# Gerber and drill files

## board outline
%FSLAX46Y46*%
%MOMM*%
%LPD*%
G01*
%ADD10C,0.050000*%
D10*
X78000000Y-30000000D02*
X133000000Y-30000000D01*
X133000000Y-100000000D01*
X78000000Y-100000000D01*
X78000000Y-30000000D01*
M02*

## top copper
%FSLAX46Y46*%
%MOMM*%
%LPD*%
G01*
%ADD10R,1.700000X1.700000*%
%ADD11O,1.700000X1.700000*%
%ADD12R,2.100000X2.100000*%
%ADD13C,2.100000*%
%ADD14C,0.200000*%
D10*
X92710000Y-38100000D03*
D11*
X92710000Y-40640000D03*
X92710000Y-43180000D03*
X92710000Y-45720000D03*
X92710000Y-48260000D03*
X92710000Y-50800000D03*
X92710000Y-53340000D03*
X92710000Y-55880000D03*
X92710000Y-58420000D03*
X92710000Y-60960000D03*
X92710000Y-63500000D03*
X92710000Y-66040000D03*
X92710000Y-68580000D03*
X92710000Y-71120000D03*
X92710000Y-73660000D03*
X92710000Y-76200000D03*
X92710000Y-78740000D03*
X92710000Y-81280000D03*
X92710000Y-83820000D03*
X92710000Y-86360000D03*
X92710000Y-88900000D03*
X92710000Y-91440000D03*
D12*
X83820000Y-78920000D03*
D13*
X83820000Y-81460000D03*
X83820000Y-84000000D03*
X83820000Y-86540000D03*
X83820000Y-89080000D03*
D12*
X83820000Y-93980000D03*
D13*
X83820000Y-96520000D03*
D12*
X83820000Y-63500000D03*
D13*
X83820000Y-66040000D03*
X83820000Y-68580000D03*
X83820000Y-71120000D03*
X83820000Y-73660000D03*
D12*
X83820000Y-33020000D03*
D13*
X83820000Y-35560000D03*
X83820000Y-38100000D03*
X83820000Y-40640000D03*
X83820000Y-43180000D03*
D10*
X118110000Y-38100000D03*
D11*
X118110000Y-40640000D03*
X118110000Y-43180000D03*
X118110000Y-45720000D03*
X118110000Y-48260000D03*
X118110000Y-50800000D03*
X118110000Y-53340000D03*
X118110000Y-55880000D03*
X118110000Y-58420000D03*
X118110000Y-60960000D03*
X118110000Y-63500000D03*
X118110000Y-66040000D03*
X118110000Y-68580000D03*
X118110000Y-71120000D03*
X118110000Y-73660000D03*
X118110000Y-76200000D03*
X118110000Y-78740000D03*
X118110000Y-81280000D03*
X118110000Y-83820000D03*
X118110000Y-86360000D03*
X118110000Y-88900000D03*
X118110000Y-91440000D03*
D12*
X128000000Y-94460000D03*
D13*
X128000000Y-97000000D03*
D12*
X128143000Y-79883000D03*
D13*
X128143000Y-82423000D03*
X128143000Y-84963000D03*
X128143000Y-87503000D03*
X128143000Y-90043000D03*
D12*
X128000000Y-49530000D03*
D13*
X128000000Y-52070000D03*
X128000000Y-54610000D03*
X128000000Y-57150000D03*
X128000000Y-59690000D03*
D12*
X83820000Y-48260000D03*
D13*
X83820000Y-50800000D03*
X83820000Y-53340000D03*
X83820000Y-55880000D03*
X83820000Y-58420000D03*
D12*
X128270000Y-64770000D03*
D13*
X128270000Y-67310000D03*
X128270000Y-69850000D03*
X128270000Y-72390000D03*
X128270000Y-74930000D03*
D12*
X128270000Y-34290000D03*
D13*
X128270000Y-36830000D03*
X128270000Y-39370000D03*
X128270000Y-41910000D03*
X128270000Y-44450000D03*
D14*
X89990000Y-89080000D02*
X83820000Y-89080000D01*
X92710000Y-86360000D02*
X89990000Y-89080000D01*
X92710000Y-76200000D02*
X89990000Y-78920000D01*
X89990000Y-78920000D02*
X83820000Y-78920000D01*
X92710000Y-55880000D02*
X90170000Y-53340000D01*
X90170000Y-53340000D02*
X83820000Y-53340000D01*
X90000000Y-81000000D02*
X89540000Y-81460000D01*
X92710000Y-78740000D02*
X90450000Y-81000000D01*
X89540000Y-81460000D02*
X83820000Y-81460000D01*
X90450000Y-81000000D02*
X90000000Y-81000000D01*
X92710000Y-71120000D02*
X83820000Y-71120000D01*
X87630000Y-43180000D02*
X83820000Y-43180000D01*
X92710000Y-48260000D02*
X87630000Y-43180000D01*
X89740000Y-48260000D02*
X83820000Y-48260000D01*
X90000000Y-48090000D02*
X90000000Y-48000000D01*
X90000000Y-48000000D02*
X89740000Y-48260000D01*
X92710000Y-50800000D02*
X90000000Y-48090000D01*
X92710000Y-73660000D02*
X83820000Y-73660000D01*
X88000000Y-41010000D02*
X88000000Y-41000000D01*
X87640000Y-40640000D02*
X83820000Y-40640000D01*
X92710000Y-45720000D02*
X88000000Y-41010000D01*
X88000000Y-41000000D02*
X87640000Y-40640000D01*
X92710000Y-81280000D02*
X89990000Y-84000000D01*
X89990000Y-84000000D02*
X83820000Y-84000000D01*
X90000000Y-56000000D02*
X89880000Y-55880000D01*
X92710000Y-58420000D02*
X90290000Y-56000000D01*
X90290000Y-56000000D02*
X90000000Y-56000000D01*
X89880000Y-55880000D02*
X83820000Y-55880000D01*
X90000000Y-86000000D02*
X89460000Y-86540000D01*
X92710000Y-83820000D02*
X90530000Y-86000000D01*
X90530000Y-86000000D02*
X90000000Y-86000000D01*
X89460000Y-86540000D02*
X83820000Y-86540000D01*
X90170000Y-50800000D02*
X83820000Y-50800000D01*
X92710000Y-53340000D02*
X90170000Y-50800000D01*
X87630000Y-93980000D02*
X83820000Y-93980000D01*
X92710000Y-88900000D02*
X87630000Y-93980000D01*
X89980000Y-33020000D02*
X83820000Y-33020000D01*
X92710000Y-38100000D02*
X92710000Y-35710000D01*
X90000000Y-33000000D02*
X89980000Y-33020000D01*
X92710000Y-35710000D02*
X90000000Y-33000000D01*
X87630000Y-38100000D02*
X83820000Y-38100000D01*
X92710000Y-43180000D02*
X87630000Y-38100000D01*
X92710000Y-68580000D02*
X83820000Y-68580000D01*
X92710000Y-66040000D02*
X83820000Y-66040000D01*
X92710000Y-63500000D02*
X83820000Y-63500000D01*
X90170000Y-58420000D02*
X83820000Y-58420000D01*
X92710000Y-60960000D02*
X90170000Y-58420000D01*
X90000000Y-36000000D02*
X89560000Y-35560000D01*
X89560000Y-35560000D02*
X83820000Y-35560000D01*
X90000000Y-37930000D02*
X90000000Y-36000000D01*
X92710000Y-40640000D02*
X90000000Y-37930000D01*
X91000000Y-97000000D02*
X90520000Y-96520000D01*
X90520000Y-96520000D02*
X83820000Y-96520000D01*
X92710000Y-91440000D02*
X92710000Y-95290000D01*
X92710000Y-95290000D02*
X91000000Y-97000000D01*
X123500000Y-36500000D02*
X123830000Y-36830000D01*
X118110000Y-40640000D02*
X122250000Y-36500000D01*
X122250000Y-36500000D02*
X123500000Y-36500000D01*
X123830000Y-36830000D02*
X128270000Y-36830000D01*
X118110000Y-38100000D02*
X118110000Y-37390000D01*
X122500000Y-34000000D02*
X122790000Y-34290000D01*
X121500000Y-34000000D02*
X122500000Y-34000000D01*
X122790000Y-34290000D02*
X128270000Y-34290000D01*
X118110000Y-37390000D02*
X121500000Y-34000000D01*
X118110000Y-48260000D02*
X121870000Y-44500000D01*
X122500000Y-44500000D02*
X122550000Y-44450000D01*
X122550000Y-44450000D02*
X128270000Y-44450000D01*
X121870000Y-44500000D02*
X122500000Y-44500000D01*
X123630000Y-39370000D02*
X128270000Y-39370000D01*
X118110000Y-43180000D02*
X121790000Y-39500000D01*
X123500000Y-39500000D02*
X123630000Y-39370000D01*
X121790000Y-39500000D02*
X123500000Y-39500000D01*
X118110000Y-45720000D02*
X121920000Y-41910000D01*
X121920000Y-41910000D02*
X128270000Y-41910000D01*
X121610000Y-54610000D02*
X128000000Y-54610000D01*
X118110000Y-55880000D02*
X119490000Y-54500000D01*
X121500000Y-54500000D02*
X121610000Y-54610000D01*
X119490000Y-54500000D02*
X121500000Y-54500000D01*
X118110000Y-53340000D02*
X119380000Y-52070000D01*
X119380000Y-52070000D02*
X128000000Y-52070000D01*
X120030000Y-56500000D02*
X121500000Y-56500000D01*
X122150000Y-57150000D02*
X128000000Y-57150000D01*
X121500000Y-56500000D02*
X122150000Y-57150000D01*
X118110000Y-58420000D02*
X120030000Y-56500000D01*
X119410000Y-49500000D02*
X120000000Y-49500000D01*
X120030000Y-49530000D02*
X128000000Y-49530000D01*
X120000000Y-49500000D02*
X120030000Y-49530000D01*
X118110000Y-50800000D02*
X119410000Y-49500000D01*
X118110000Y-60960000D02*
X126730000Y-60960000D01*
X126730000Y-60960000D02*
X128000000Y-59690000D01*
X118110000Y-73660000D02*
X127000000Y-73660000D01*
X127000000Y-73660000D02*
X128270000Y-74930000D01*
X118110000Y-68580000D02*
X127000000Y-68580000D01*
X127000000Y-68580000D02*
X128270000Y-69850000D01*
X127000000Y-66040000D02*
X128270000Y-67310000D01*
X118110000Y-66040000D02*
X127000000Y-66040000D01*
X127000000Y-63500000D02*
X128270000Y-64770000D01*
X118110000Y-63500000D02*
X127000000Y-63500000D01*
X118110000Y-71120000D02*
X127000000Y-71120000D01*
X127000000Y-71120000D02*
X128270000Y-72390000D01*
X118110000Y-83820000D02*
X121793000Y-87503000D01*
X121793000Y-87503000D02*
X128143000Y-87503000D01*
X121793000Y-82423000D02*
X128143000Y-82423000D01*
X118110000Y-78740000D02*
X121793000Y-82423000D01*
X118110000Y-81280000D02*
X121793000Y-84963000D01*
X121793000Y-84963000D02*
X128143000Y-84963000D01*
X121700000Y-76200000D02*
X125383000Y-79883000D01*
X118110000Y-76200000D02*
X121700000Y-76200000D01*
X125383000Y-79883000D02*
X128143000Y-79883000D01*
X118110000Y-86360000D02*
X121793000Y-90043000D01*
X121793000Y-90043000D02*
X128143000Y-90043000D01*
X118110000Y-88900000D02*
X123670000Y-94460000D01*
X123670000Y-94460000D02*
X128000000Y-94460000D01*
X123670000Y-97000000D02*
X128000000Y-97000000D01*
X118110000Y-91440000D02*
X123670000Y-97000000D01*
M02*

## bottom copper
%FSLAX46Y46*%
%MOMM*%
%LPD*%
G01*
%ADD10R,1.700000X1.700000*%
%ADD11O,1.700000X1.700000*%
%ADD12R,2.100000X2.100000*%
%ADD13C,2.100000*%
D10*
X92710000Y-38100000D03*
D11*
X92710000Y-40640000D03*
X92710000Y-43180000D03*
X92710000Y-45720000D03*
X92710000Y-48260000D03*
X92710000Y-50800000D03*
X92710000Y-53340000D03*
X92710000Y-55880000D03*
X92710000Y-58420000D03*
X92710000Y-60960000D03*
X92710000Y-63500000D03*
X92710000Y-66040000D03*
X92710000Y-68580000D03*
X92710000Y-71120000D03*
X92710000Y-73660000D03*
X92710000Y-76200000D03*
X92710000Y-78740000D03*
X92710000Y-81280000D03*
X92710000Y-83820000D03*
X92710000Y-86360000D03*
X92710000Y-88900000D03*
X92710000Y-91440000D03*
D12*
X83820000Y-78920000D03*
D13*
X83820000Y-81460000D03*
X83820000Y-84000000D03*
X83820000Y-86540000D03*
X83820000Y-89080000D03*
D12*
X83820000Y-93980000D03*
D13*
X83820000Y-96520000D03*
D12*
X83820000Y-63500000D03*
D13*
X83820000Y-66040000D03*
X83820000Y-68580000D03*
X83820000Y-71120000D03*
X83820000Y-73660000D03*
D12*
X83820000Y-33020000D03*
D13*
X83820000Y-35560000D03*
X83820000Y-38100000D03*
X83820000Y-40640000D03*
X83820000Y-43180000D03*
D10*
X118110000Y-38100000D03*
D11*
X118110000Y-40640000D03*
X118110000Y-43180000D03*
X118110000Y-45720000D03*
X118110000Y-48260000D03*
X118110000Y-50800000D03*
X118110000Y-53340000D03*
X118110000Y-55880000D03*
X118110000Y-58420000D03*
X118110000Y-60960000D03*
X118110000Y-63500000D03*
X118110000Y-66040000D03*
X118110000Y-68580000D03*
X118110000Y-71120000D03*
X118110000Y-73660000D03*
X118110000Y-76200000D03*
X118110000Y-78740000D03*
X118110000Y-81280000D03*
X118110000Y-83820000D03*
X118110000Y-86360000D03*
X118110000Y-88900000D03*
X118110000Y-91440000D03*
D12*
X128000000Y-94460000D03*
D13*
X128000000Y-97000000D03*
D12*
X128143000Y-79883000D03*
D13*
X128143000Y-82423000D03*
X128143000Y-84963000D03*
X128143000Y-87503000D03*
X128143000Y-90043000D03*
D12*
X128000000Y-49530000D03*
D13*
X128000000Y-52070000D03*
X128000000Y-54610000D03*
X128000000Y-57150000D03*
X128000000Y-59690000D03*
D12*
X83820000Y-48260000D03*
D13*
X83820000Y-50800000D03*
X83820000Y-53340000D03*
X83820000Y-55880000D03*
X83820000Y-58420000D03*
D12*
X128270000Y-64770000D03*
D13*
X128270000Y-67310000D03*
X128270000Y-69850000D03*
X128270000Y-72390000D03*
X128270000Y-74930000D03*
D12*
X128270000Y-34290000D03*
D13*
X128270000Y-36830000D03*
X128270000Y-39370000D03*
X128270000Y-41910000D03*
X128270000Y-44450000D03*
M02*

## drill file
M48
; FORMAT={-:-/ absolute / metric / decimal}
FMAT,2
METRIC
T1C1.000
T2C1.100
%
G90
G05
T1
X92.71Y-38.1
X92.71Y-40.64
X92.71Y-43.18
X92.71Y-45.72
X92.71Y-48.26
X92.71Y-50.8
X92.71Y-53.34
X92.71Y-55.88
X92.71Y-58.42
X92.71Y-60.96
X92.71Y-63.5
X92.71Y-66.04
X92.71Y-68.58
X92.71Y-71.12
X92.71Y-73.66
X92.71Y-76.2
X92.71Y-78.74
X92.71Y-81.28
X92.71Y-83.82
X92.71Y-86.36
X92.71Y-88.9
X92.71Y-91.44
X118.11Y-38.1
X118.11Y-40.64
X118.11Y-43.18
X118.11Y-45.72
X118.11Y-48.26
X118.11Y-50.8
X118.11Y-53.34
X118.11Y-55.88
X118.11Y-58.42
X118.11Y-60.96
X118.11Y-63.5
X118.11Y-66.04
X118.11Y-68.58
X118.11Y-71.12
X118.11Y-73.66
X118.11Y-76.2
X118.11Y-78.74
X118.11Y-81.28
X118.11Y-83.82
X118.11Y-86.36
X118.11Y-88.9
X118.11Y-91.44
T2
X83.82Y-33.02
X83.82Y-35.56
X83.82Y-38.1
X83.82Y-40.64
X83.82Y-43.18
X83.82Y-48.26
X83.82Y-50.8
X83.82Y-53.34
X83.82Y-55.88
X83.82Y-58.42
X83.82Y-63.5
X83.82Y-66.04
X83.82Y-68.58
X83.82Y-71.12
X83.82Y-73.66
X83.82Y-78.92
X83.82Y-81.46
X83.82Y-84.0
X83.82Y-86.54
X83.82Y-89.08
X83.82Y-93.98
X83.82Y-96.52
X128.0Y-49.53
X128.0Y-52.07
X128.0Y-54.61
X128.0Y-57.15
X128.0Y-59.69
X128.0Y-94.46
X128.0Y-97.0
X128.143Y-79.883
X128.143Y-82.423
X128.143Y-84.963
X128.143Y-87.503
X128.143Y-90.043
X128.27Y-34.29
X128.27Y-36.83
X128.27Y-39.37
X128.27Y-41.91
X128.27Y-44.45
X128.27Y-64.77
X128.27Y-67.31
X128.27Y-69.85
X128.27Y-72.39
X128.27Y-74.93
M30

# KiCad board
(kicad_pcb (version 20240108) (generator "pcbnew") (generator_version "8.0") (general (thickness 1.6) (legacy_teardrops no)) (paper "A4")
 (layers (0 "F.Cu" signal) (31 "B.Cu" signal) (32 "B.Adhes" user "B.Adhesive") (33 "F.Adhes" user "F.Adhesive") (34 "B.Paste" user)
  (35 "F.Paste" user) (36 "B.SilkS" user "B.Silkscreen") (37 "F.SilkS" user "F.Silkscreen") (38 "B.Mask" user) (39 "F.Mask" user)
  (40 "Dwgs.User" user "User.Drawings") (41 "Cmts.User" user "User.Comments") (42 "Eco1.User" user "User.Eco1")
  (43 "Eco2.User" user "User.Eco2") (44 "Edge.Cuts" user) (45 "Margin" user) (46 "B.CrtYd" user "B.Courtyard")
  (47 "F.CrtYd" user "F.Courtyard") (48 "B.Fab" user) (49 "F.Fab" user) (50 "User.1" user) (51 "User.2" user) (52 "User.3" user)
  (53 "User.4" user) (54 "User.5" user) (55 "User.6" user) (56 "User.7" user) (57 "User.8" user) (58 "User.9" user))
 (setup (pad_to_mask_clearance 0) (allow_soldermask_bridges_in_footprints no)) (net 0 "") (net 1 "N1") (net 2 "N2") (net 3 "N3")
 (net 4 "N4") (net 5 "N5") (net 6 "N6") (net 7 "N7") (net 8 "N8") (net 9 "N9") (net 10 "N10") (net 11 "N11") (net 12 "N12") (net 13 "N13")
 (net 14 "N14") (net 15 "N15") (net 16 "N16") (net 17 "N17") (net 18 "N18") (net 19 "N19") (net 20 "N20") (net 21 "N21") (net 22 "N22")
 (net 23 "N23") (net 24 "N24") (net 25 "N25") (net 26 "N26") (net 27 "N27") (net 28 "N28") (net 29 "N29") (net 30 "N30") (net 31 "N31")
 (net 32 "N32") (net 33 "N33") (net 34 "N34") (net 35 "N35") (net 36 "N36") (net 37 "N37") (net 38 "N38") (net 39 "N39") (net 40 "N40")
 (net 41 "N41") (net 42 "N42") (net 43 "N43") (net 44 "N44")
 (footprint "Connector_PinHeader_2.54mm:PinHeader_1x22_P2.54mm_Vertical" (layer "F.Cu") (at 92.71 38.1)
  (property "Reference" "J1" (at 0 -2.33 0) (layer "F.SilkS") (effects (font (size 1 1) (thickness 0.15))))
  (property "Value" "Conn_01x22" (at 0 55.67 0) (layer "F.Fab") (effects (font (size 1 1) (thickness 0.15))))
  (pad "1" thru_hole rect (at 0 0) (size 1.7 1.7) (drill 1) (layers "*.Cu" "*.Mask") (remove_unused_layers no) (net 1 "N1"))
  (pad "2" thru_hole oval (at 0 2.54) (size 1.7 1.7) (drill 1) (layers "*.Cu" "*.Mask") (remove_unused_layers no) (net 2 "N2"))
  (pad "3" thru_hole oval (at 0 5.08) (size 1.7 1.7) (drill 1) (layers "*.Cu" "*.Mask") (remove_unused_layers no) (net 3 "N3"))
  (pad "4" thru_hole oval (at 0 7.62) (size 1.7 1.7) (drill 1) (layers "*.Cu" "*.Mask") (remove_unused_layers no) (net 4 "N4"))
  (pad "5" thru_hole oval (at 0 10.16) (size 1.7 1.7) (drill 1) (layers "*.Cu" "*.Mask") (remove_unused_layers no) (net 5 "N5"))
  (pad "6" thru_hole oval (at 0 12.7) (size 1.7 1.7) (drill 1) (layers "*.Cu" "*.Mask") (remove_unused_layers no) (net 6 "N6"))
  (pad "7" thru_hole oval (at 0 15.24) (size 1.7 1.7) (drill 1) (layers "*.Cu" "*.Mask") (remove_unused_layers no) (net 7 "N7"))
  (pad "8" thru_hole oval (at 0 17.78) (size 1.7 1.7) (drill 1) (layers "*.Cu" "*.Mask") (remove_unused_layers no) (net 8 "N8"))
  (pad "9" thru_hole oval (at 0 20.32) (size 1.7 1.7) (drill 1) (layers "*.Cu" "*.Mask") (remove_unused_layers no) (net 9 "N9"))
  (pad "10" thru_hole oval (at 0 22.86) (size 1.7 1.7) (drill 1) (layers "*.Cu" "*.Mask") (remove_unused_layers no) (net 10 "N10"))
  (pad "11" thru_hole oval (at 0 25.4) (size 1.7 1.7) (drill 1) (layers "*.Cu" "*.Mask") (remove_unused_layers no) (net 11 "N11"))
  (pad "12" thru_hole oval (at 0 27.94) (size 1.7 1.7) (drill 1) (layers "*.Cu" "*.Mask") (remove_unused_layers no) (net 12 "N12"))
  (pad "13" thru_hole oval (at 0 30.48) (size 1.7 1.7) (drill 1) (layers "*.Cu" "*.Mask") (remove_unused_layers no) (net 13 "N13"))
  (pad "14" thru_hole oval (at 0 33.02) (size 1.7 1.7) (drill 1) (layers "*.Cu" "*.Mask") (remove_unused_layers no) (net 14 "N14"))
  (pad "15" thru_hole oval (at 0 35.56) (size 1.7 1.7) (drill 1) (layers "*.Cu" "*.Mask") (remove_unused_layers no) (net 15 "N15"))
  (pad "16" thru_hole oval (at 0 38.1) (size 1.7 1.7) (drill 1) (layers "*.Cu" "*.Mask") (remove_unused_layers no) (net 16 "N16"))
  (pad "17" thru_hole oval (at 0 40.64) (size 1.7 1.7) (drill 1) (layers "*.Cu" "*.Mask") (remove_unused_layers no) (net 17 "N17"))
  (pad "18" thru_hole oval (at 0 43.18) (size 1.7 1.7) (drill 1) (layers "*.Cu" "*.Mask") (remove_unused_layers no) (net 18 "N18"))
  (pad "19" thru_hole oval (at 0 45.72) (size 1.7 1.7) (drill 1) (layers "*.Cu" "*.Mask") (remove_unused_layers no) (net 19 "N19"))
  (pad "20" thru_hole oval (at 0 48.26) (size 1.7 1.7) (drill 1) (layers "*.Cu" "*.Mask") (remove_unused_layers no) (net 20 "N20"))
  (pad "21" thru_hole oval (at 0 50.8) (size 1.7 1.7) (drill 1) (layers "*.Cu" "*.Mask") (remove_unused_layers no) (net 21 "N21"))
  (pad "22" thru_hole oval (at 0 53.34) (size 1.7 1.7) (drill 1) (layers "*.Cu" "*.Mask") (remove_unused_layers no) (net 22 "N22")))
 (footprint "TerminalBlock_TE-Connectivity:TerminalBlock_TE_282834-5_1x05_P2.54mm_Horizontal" (layer "F.Cu") (at 83.82 78.92 -90)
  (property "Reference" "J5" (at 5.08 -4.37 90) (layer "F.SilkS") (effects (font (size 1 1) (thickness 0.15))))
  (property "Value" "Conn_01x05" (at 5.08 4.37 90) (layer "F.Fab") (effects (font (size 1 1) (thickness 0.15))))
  (pad "1" thru_hole rect (at 0 0 270) (size 2.1 2.1) (drill 1.1) (layers "*.Cu" "*.Mask") (remove_unused_layers no) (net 16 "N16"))
  (pad "2" thru_hole circle (at 2.54 0 270) (size 2.1 2.1) (drill 1.1) (layers "*.Cu" "*.Mask") (remove_unused_layers no) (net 17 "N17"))
  (pad "3" thru_hole circle (at 5.08 0 270) (size 2.1 2.1) (drill 1.1) (layers "*.Cu" "*.Mask") (remove_unused_layers no) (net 18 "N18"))
  (pad "4" thru_hole circle (at 7.62 0 270) (size 2.1 2.1) (drill 1.1) (layers "*.Cu" "*.Mask") (remove_unused_layers no) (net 19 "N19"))
  (pad "5" thru_hole circle (at 10.16 0 270) (size 2.1 2.1) (drill 1.1) (layers "*.Cu" "*.Mask") (remove_unused_layers no) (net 20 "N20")))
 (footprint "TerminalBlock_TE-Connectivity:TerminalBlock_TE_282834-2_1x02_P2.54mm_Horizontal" (layer "F.Cu") (at 83.82 93.98 -90)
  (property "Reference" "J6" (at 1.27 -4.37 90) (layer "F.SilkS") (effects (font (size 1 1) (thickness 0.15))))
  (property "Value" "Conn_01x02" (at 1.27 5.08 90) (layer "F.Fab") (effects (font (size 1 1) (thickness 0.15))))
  (pad "1" thru_hole rect (at 0 0 270) (size 2.1 2.1) (drill 1.1) (layers "*.Cu" "*.Mask") (remove_unused_layers no) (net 21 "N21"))
  (pad "2" thru_hole circle (at 2.54 0 270) (size 2.1 2.1) (drill 1.1) (layers "*.Cu" "*.Mask") (remove_unused_layers no) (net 22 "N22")))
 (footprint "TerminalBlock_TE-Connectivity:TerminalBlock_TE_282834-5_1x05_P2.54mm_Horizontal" (layer "F.Cu") (at 83.82 63.5 -90)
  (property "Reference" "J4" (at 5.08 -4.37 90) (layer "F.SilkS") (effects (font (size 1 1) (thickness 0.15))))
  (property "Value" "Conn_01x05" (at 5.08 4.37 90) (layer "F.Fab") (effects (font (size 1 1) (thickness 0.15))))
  (pad "1" thru_hole rect (at 0 0 270) (size 2.1 2.1) (drill 1.1) (layers "*.Cu" "*.Mask") (remove_unused_layers no) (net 11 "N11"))
  (pad "2" thru_hole circle (at 2.54 0 270) (size 2.1 2.1) (drill 1.1) (layers "*.Cu" "*.Mask") (remove_unused_layers no) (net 12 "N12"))
  (pad "3" thru_hole circle (at 5.08 0 270) (size 2.1 2.1) (drill 1.1) (layers "*.Cu" "*.Mask") (remove_unused_layers no) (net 13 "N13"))
  (pad "4" thru_hole circle (at 7.62 0 270) (size 2.1 2.1) (drill 1.1) (layers "*.Cu" "*.Mask") (remove_unused_layers no) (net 14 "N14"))
  (pad "5" thru_hole circle (at 10.16 0 270) (size 2.1 2.1) (drill 1.1) (layers "*.Cu" "*.Mask") (remove_unused_layers no) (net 15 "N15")))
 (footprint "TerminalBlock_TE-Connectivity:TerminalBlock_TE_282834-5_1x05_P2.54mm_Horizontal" (layer "F.Cu") (at 83.82 33.02 -90)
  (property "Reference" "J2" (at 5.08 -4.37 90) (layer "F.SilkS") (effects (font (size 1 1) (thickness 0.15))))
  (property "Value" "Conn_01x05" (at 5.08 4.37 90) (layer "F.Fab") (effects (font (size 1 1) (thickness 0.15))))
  (pad "1" thru_hole rect (at 0 0 270) (size 2.1 2.1) (drill 1.1) (layers "*.Cu" "*.Mask") (remove_unused_layers no) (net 1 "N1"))
  (pad "2" thru_hole circle (at 2.54 0 270) (size 2.1 2.1) (drill 1.1) (layers "*.Cu" "*.Mask") (remove_unused_layers no) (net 2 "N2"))
  (pad "3" thru_hole circle (at 5.08 0 270) (size 2.1 2.1) (drill 1.1) (layers "*.Cu" "*.Mask") (remove_unused_layers no) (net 3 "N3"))
  (pad "4" thru_hole circle (at 7.62 0 270) (size 2.1 2.1) (drill 1.1) (layers "*.Cu" "*.Mask") (remove_unused_layers no) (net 4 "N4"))
  (pad "5" thru_hole circle (at 10.16 0 270) (size 2.1 2.1) (drill 1.1) (layers "*.Cu" "*.Mask") (remove_unused_layers no) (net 5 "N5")))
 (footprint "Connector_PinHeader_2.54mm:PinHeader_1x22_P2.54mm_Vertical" (layer "F.Cu") (at 118.11 38.1)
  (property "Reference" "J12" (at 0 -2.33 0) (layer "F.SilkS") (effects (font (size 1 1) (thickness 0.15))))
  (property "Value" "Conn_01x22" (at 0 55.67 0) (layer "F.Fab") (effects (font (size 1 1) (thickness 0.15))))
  (pad "1" thru_hole rect (at 0 0) (size 1.7 1.7) (drill 1) (layers "*.Cu" "*.Mask") (remove_unused_layers no) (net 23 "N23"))
  (pad "2" thru_hole oval (at 0 2.54) (size 1.7 1.7) (drill 1) (layers "*.Cu" "*.Mask") (remove_unused_layers no) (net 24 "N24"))
  (pad "3" thru_hole oval (at 0 5.08) (size 1.7 1.7) (drill 1) (layers "*.Cu" "*.Mask") (remove_unused_layers no) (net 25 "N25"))
  (pad "4" thru_hole oval (at 0 7.62) (size 1.7 1.7) (drill 1) (layers "*.Cu" "*.Mask") (remove_unused_layers no) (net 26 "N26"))
  (pad "5" thru_hole oval (at 0 10.16) (size 1.7 1.7) (drill 1) (layers "*.Cu" "*.Mask") (remove_unused_layers no) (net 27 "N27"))
  (pad "6" thru_hole oval (at 0 12.7) (size 1.7 1.7) (drill 1) (layers "*.Cu" "*.Mask") (remove_unused_layers no) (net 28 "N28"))
  (pad "7" thru_hole oval (at 0 15.24) (size 1.7 1.7) (drill 1) (layers "*.Cu" "*.Mask") (remove_unused_layers no) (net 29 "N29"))
  (pad "8" thru_hole oval (at 0 17.78) (size 1.7 1.7) (drill 1) (layers "*.Cu" "*.Mask") (remove_unused_layers no) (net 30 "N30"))
  (pad "9" thru_hole oval (at 0 20.32) (size 1.7 1.7) (drill 1) (layers "*.Cu" "*.Mask") (remove_unused_layers no) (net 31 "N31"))
  (pad "10" thru_hole oval (at 0 22.86) (size 1.7 1.7) (drill 1) (layers "*.Cu" "*.Mask") (remove_unused_layers no) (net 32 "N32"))
  (pad "11" thru_hole oval (at 0 25.4) (size 1.7 1.7) (drill 1) (layers "*.Cu" "*.Mask") (remove_unused_layers no) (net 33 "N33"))
  (pad "12" thru_hole oval (at 0 27.94) (size 1.7 1.7) (drill 1) (layers "*.Cu" "*.Mask") (remove_unused_layers no) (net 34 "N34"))
  (pad "13" thru_hole oval (at 0 30.48) (size 1.7 1.7) (drill 1) (layers "*.Cu" "*.Mask") (remove_unused_layers no) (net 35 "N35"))
  (pad "14" thru_hole oval (at 0 33.02) (size 1.7 1.7) (drill 1) (layers "*.Cu" "*.Mask") (remove_unused_layers no) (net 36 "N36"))
  (pad "15" thru_hole oval (at 0 35.56) (size 1.7 1.7) (drill 1) (layers "*.Cu" "*.Mask") (remove_unused_layers no) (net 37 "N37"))
  (pad "16" thru_hole oval (at 0 38.1) (size 1.7 1.7) (drill 1) (layers "*.Cu" "*.Mask") (remove_unused_layers no) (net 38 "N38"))
  (pad "17" thru_hole oval (at 0 40.64) (size 1.7 1.7) (drill 1) (layers "*.Cu" "*.Mask") (remove_unused_layers no) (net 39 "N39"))
  (pad "18" thru_hole oval (at 0 43.18) (size 1.7 1.7) (drill 1) (layers "*.Cu" "*.Mask") (remove_unused_layers no) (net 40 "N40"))
  (pad "19" thru_hole oval (at 0 45.72) (size 1.7 1.7) (drill 1) (layers "*.Cu" "*.Mask") (remove_unused_layers no) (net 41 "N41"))
  (pad "20" thru_hole oval (at 0 48.26) (size 1.7 1.7) (drill 1) (layers "*.Cu" "*.Mask") (remove_unused_layers no) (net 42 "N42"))
  (pad "21" thru_hole oval (at 0 50.8) (size 1.7 1.7) (drill 1) (layers "*.Cu" "*.Mask") (remove_unused_layers no) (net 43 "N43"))
  (pad "22" thru_hole oval (at 0 53.34) (size 1.7 1.7) (drill 1) (layers "*.Cu" "*.Mask") (remove_unused_layers no) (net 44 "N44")))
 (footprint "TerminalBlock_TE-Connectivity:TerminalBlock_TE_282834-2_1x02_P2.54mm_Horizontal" (layer "F.Cu") (at 128 94.46 -90)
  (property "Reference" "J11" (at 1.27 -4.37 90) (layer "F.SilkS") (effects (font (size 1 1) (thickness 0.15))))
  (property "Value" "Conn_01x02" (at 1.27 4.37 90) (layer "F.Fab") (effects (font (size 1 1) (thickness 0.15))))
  (pad "1" thru_hole rect (at 0 0 270) (size 2.1 2.1) (drill 1.1) (layers "*.Cu" "*.Mask") (remove_unused_layers no) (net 43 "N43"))
  (pad "2" thru_hole circle (at 2.54 0 270) (size 2.1 2.1) (drill 1.1) (layers "*.Cu" "*.Mask") (remove_unused_layers no) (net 44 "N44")))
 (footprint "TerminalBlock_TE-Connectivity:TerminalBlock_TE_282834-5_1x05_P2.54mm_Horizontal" (layer "F.Cu") (at 128.143 79.883 -90)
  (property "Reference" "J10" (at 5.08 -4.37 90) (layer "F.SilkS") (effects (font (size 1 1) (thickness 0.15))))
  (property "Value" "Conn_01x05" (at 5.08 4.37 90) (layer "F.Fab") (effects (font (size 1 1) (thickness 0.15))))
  (pad "1" thru_hole rect (at 0 0 270) (size 2.1 2.1) (drill 1.1) (layers "*.Cu" "*.Mask") (remove_unused_layers no) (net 38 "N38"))
  (pad "2" thru_hole circle (at 2.54 0 270) (size 2.1 2.1) (drill 1.1) (layers "*.Cu" "*.Mask") (remove_unused_layers no) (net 39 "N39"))
  (pad "3" thru_hole circle (at 5.08 0 270) (size 2.1 2.1) (drill 1.1) (layers "*.Cu" "*.Mask") (remove_unused_layers no) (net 40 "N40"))
  (pad "4" thru_hole circle (at 7.62 0 270) (size 2.1 2.1) (drill 1.1) (layers "*.Cu" "*.Mask") (remove_unused_layers no) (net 41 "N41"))
  (pad "5" thru_hole circle (at 10.16 0 270) (size 2.1 2.1) (drill 1.1) (layers "*.Cu" "*.Mask") (remove_unused_layers no) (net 42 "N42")))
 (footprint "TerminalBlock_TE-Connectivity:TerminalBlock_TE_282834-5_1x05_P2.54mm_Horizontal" (layer "F.Cu") (at 128 49.53 -90)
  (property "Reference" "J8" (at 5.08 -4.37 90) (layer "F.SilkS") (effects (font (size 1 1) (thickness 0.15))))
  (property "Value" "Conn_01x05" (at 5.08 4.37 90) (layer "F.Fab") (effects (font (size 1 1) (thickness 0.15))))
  (pad "1" thru_hole rect (at 0 0 270) (size 2.1 2.1) (drill 1.1) (layers "*.Cu" "*.Mask") (remove_unused_layers no) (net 28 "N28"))
  (pad "2" thru_hole circle (at 2.54 0 270) (size 2.1 2.1) (drill 1.1) (layers "*.Cu" "*.Mask") (remove_unused_layers no) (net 29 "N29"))
  (pad "3" thru_hole circle (at 5.08 0 270) (size 2.1 2.1) (drill 1.1) (layers "*.Cu" "*.Mask") (remove_unused_layers no) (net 30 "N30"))
  (pad "4" thru_hole circle (at 7.62 0 270) (size 2.1 2.1) (drill 1.1) (layers "*.Cu" "*.Mask") (remove_unused_layers no) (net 31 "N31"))
  (pad "5" thru_hole circle (at 10.16 0 270) (size 2.1 2.1) (drill 1.1) (layers "*.Cu" "*.Mask") (remove_unused_layers no) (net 32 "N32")))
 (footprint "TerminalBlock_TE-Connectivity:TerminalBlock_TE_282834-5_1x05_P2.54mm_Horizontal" (layer "F.Cu") (at 83.82 48.26 -90)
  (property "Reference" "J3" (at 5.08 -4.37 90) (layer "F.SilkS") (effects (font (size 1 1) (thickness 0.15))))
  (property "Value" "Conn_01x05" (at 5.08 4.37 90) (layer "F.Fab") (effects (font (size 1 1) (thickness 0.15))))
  (pad "1" thru_hole rect (at 0 0 270) (size 2.1 2.1) (drill 1.1) (layers "*.Cu" "*.Mask") (remove_unused_layers no) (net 6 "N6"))
  (pad "2" thru_hole circle (at 2.54 0 270) (size 2.1 2.1) (drill 1.1) (layers "*.Cu" "*.Mask") (remove_unused_layers no) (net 7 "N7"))
  (pad "3" thru_hole circle (at 5.08 0 270) (size 2.1 2.1) (drill 1.1) (layers "*.Cu" "*.Mask") (remove_unused_layers no) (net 8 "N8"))
  (pad "4" thru_hole circle (at 7.62 0 270) (size 2.1 2.1) (drill 1.1) (layers "*.Cu" "*.Mask") (remove_unused_layers no) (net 9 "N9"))
  (pad "5" thru_hole circle (at 10.16 0 270) (size 2.1 2.1) (drill 1.1) (layers "*.Cu" "*.Mask") (remove_unused_layers no) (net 10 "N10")))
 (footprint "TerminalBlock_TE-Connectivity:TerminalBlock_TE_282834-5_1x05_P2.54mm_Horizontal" (layer "F.Cu") (at 128.27 64.77 -90)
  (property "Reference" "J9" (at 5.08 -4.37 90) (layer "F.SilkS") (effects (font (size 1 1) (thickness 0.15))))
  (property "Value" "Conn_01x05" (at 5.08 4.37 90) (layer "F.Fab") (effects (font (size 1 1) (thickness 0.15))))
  (pad "1" thru_hole rect (at 0 0 270) (size 2.1 2.1) (drill 1.1) (layers "*.Cu" "*.Mask") (remove_unused_layers no) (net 33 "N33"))
  (pad "2" thru_hole circle (at 2.54 0 270) (size 2.1 2.1) (drill 1.1) (layers "*.Cu" "*.Mask") (remove_unused_layers no) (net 34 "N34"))
  (pad "3" thru_hole circle (at 5.08 0 270) (size 2.1 2.1) (drill 1.1) (layers "*.Cu" "*.Mask") (remove_unused_layers no) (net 35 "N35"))
  (pad "4" thru_hole circle (at 7.62 0 270) (size 2.1 2.1) (drill 1.1) (layers "*.Cu" "*.Mask") (remove_unused_layers no) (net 36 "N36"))
  (pad "5" thru_hole circle (at 10.16 0 270) (size 2.1 2.1) (drill 1.1) (layers "*.Cu" "*.Mask") (remove_unused_layers no) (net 37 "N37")))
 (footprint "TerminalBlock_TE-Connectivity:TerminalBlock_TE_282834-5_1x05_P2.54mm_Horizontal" (layer "F.Cu") (at 128.27 34.29 -90)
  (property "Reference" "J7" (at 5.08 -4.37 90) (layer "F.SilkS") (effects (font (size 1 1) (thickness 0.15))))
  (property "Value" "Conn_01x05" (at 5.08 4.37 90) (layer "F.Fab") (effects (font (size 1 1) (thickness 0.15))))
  (pad "1" thru_hole rect (at 0 0 270) (size 2.1 2.1) (drill 1.1) (layers "*.Cu" "*.Mask") (remove_unused_layers no) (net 23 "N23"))
  (pad "2" thru_hole circle (at 2.54 0 270) (size 2.1 2.1) (drill 1.1) (layers "*.Cu" "*.Mask") (remove_unused_layers no) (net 24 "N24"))
  (pad "3" thru_hole circle (at 5.08 0 270) (size 2.1 2.1) (drill 1.1) (layers "*.Cu" "*.Mask") (remove_unused_layers no) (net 25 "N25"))
  (pad "4" thru_hole circle (at 7.62 0 270) (size 2.1 2.1) (drill 1.1) (layers "*.Cu" "*.Mask") (remove_unused_layers no) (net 26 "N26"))
  (pad "5" thru_hole circle (at 10.16 0 270) (size 2.1 2.1) (drill 1.1) (layers "*.Cu" "*.Mask") (remove_unused_layers no) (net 27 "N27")))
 (gr_rect (start 78 30) (end 133 100) (stroke (width 0.05) (type default)) (fill none) (layer "Edge.Cuts"))
 (segment (start 89.99 89.08) (end 83.82 89.08) (width 0.2) (layer "F.Cu") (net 20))
 (segment (start 92.71 86.36) (end 89.99 89.08) (width 0.2) (layer "F.Cu") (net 20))
 (segment (start 92.71 76.2) (end 89.99 78.92) (width 0.2) (layer "F.Cu") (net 16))
 (segment (start 89.99 78.92) (end 83.82 78.92) (width 0.2) (layer "F.Cu") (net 16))
 (segment (start 92.71 55.88) (end 90.17 53.34) (width 0.2) (layer "F.Cu") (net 8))
 (segment (start 90.17 53.34) (end 83.82 53.34) (width 0.2) (layer "F.Cu") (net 8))
 (segment (start 90 81) (end 89.54 81.46) (width 0.2) (layer "F.Cu") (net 17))
 (segment (start 92.71 78.74) (end 90.45 81) (width 0.2) (layer "F.Cu") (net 17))
 (segment (start 89.54 81.46) (end 83.82 81.46) (width 0.2) (layer "F.Cu") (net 17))
 (segment (start 90.45 81) (end 90 81) (width 0.2) (layer "F.Cu") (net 17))
 (segment (start 92.71 71.12) (end 83.82 71.12) (width 0.2) (layer "F.Cu") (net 14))
 (segment (start 87.63 43.18) (end 83.82 43.18) (width 0.2) (layer "F.Cu") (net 5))
 (segment (start 92.71 48.26) (end 87.63 43.18) (width 0.2) (layer "F.Cu") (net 5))
 (segment (start 89.74 48.26) (end 83.82 48.26) (width 0.2) (layer "F.Cu") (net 6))
 (segment (start 90 48.09) (end 90 48) (width 0.2) (layer "F.Cu") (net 6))
 (segment (start 90 48) (end 89.74 48.26) (width 0.2) (layer "F.Cu") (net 6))
 (segment (start 92.71 50.8) (end 90 48.09) (width 0.2) (layer "F.Cu") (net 6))
 (segment (start 92.71 73.66) (end 83.82 73.66) (width 0.2) (layer "F.Cu") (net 15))
 (segment (start 88 41.01) (end 88 41) (width 0.2) (layer "F.Cu") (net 4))
 (segment (start 87.64 40.64) (end 83.82 40.64) (width 0.2) (layer "F.Cu") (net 4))
 (segment (start 92.71 45.72) (end 88 41.01) (width 0.2) (layer "F.Cu") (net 4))
 (segment (start 88 41) (end 87.64 40.64) (width 0.2) (layer "F.Cu") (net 4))
 (segment (start 92.71 81.28) (end 89.99 84) (width 0.2) (layer "F.Cu") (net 18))
 (segment (start 89.99 84) (end 83.82 84) (width 0.2) (layer "F.Cu") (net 18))
 (segment (start 90 56) (end 89.88 55.88) (width 0.2) (layer "F.Cu") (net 9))
 (segment (start 92.71 58.42) (end 90.29 56) (width 0.2) (layer "F.Cu") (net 9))
 (segment (start 90.29 56) (end 90 56) (width 0.2) (layer "F.Cu") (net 9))
 (segment (start 89.88 55.88) (end 83.82 55.88) (width 0.2) (layer "F.Cu") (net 9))
 (segment (start 90 86) (end 89.46 86.54) (width 0.2) (layer "F.Cu") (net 19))
 (segment (start 92.71 83.82) (end 90.53 86) (width 0.2) (layer "F.Cu") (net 19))
 (segment (start 90.53 86) (end 90 86) (width 0.2) (layer "F.Cu") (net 19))
 (segment (start 89.46 86.54) (end 83.82 86.54) (width 0.2) (layer "F.Cu") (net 19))
 (segment (start 90.17 50.8) (end 83.82 50.8) (width 0.2) (layer "F.Cu") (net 7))
 (segment (start 92.71 53.34) (end 90.17 50.8) (width 0.2) (layer "F.Cu") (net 7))
 (segment (start 87.63 93.98) (end 83.82 93.98) (width 0.2) (layer "F.Cu") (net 21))
 (segment (start 92.71 88.9) (end 87.63 93.98) (width 0.2) (layer "F.Cu") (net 21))
 (segment (start 89.98 33.02) (end 83.82 33.02) (width 0.2) (layer "F.Cu") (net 1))
 (segment (start 92.71 38.1) (end 92.71 35.71) (width 0.2) (layer "F.Cu") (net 1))
 (segment (start 90 33) (end 89.98 33.02) (width 0.2) (layer "F.Cu") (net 1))
 (segment (start 92.71 35.71) (end 90 33) (width 0.2) (layer "F.Cu") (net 1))
 (segment (start 87.63 38.1) (end 83.82 38.1) (width 0.2) (layer "F.Cu") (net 3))
 (segment (start 92.71 43.18) (end 87.63 38.1) (width 0.2) (layer "F.Cu") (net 3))
 (segment (start 92.71 68.58) (end 83.82 68.58) (width 0.2) (layer "F.Cu") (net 13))
 (segment (start 92.71 66.04) (end 83.82 66.04) (width 0.2) (layer "F.Cu") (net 12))
 (segment (start 92.71 63.5) (end 83.82 63.5) (width 0.2) (layer "F.Cu") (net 11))
 (segment (start 90.17 58.42) (end 83.82 58.42) (width 0.2) (layer "F.Cu") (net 10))
 (segment (start 92.71 60.96) (end 90.17 58.42) (width 0.2) (layer "F.Cu") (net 10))
 (segment (start 90 36) (end 89.56 35.56) (width 0.2) (layer "F.Cu") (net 2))
 (segment (start 89.56 35.56) (end 83.82 35.56) (width 0.2) (layer "F.Cu") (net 2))
 (segment (start 90 37.93) (end 90 36) (width 0.2) (layer "F.Cu") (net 2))
 (segment (start 92.71 40.64) (end 90 37.93) (width 0.2) (layer "F.Cu") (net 2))
 (segment (start 91 97) (end 90.52 96.52) (width 0.2) (layer "F.Cu") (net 22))
 (segment (start 90.52 96.52) (end 83.82 96.52) (width 0.2) (layer "F.Cu") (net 22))
 (segment (start 92.71 91.44) (end 92.71 95.29) (width 0.2) (layer "F.Cu") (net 22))
 (segment (start 92.71 95.29) (end 91 97) (width 0.2) (layer "F.Cu") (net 22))
 (segment (start 123.5 36.5) (end 123.83 36.83) (width 0.2) (layer "F.Cu") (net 24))
 (segment (start 118.11 40.64) (end 122.25 36.5) (width 0.2) (layer "F.Cu") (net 24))
 (segment (start 122.25 36.5) (end 123.5 36.5) (width 0.2) (layer "F.Cu") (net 24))
 (segment (start 123.83 36.83) (end 128.27 36.83) (width 0.2) (layer "F.Cu") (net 24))
 (segment (start 118.11 38.1) (end 118.11 37.39) (width 0.2) (layer "F.Cu") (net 23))
 (segment (start 122.5 34) (end 122.79 34.29) (width 0.2) (layer "F.Cu") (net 23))
 (segment (start 121.5 34) (end 122.5 34) (width 0.2) (layer "F.Cu") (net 23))
 (segment (start 122.79 34.29) (end 128.27 34.29) (width 0.2) (layer "F.Cu") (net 23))
 (segment (start 118.11 37.39) (end 121.5 34) (width 0.2) (layer "F.Cu") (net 23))
 (segment (start 118.11 48.26) (end 121.87 44.5) (width 0.2) (layer "F.Cu") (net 27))
 (segment (start 122.5 44.5) (end 122.55 44.45) (width 0.2) (layer "F.Cu") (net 27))
 (segment (start 122.55 44.45) (end 128.27 44.45) (width 0.2) (layer "F.Cu") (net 27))
 (segment (start 121.87 44.5) (end 122.5 44.5) (width 0.2) (layer "F.Cu") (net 27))
 (segment (start 123.63 39.37) (end 128.27 39.37) (width 0.2) (layer "F.Cu") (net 25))
 (segment (start 118.11 43.18) (end 121.79 39.5) (width 0.2) (layer "F.Cu") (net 25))
 (segment (start 123.5 39.5) (end 123.63 39.37) (width 0.2) (layer "F.Cu") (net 25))
 (segment (start 121.79 39.5) (end 123.5 39.5) (width 0.2) (layer "F.Cu") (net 25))
 (segment (start 118.11 45.72) (end 121.92 41.91) (width 0.2) (layer "F.Cu") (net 26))
 (segment (start 121.92 41.91) (end 128.27 41.91) (width 0.2) (layer "F.Cu") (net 26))
 (segment (start 121.61 54.61) (end 128 54.61) (width 0.2) (layer "F.Cu") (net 30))
 (segment (start 118.11 55.88) (end 119.49 54.5) (width 0.2) (layer "F.Cu") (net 30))
 (segment (start 121.5 54.5) (end 121.61 54.61) (width 0.2) (layer "F.Cu") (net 30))
 (segment (start 119.49 54.5) (end 121.5 54.5) (width 0.2) (layer "F.Cu") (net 30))
 (segment (start 118.11 53.34) (end 119.38 52.07) (width 0.2) (layer "F.Cu") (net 29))
 (segment (start 119.38 52.07) (end 128 52.07) (width 0.2) (layer "F.Cu") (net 29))
 (segment (start 120.03 56.5) (end 121.5 56.5) (width 0.2) (layer "F.Cu") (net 31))
 (segment (start 122.15 57.15) (end 128 57.15) (width 0.2) (layer "F.Cu") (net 31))
 (segment (start 121.5 56.5) (end 122.15 57.15) (width 0.2) (layer "F.Cu") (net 31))
 (segment (start 118.11 58.42) (end 120.03 56.5) (width 0.2) (layer "F.Cu") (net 31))
 (segment (start 119.41 49.5) (end 120 49.5) (width 0.2) (layer "F.Cu") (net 28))
 (segment (start 120.03 49.53) (end 128 49.53) (width 0.2) (layer "F.Cu") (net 28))
 (segment (start 120 49.5) (end 120.03 49.53) (width 0.2) (layer "F.Cu") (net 28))
 (segment (start 118.11 50.8) (end 119.41 49.5) (width 0.2) (layer "F.Cu") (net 28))
 (segment (start 118.11 60.96) (end 126.73 60.96) (width 0.2) (layer "F.Cu") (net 32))
 (segment (start 126.73 60.96) (end 128 59.69) (width 0.2) (layer "F.Cu") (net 32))
 (segment (start 118.11 73.66) (end 127 73.66) (width 0.2) (layer "F.Cu") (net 37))
 (segment (start 127 73.66) (end 128.27 74.93) (width 0.2) (layer "F.Cu") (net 37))
 (segment (start 118.11 68.58) (end 127 68.58) (width 0.2) (layer "F.Cu") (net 35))
 (segment (start 127 68.58) (end 128.27 69.85) (width 0.2) (layer "F.Cu") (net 35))
 (segment (start 127 66.04) (end 128.27 67.31) (width 0.2) (layer "F.Cu") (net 34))
 (segment (start 118.11 66.04) (end 127 66.04) (width 0.2) (layer "F.Cu") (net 34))
 (segment (start 127 63.5) (end 128.27 64.77) (width 0.2) (layer "F.Cu") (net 33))
 (segment (start 118.11 63.5) (end 127 63.5) (width 0.2) (layer "F.Cu") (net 33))
 (segment (start 118.11 71.12) (end 127 71.12) (width 0.2) (layer "F.Cu") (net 36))
 (segment (start 127 71.12) (end 128.27 72.39) (width 0.2) (layer "F.Cu") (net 36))
 (segment (start 118.11 83.82) (end 121.793 87.503) (width 0.2) (layer "F.Cu") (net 41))
 (segment (start 121.793 87.503) (end 128.143 87.503) (width 0.2) (layer "F.Cu") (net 41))
 (segment (start 121.793 82.423) (end 128.143 82.423) (width 0.2) (layer "F.Cu") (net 39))
 (segment (start 118.11 78.74) (end 121.793 82.423) (width 0.2) (layer "F.Cu") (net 39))
 (segment (start 118.11 81.28) (end 121.793 84.963) (width 0.2) (layer "F.Cu") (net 40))
 (segment (start 121.793 84.963) (end 128.143 84.963) (width 0.2) (layer "F.Cu") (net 40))
 (segment (start 121.7 76.2) (end 125.383 79.883) (width 0.2) (layer "F.Cu") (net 38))
 (segment (start 118.11 76.2) (end 121.7 76.2) (width 0.2) (layer "F.Cu") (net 38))
 (segment (start 125.383 79.883) (end 128.143 79.883) (width 0.2) (layer "F.Cu") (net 38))
 (segment (start 118.11 86.36) (end 121.793 90.043) (width 0.2) (layer "F.Cu") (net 42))
 (segment (start 121.793 90.043) (end 128.143 90.043) (width 0.2) (layer "F.Cu") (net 42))
 (segment (start 118.11 88.9) (end 123.67 94.46) (width 0.2) (layer "F.Cu") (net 43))
 (segment (start 123.67 94.46) (end 128 94.46) (width 0.2) (layer "F.Cu") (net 43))
 (segment (start 123.67 97) (end 128 97) (width 0.2) (layer "F.Cu") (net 44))
 (segment (start 118.11 91.44) (end 123.67 97) (width 0.2) (layer "F.Cu") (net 44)))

